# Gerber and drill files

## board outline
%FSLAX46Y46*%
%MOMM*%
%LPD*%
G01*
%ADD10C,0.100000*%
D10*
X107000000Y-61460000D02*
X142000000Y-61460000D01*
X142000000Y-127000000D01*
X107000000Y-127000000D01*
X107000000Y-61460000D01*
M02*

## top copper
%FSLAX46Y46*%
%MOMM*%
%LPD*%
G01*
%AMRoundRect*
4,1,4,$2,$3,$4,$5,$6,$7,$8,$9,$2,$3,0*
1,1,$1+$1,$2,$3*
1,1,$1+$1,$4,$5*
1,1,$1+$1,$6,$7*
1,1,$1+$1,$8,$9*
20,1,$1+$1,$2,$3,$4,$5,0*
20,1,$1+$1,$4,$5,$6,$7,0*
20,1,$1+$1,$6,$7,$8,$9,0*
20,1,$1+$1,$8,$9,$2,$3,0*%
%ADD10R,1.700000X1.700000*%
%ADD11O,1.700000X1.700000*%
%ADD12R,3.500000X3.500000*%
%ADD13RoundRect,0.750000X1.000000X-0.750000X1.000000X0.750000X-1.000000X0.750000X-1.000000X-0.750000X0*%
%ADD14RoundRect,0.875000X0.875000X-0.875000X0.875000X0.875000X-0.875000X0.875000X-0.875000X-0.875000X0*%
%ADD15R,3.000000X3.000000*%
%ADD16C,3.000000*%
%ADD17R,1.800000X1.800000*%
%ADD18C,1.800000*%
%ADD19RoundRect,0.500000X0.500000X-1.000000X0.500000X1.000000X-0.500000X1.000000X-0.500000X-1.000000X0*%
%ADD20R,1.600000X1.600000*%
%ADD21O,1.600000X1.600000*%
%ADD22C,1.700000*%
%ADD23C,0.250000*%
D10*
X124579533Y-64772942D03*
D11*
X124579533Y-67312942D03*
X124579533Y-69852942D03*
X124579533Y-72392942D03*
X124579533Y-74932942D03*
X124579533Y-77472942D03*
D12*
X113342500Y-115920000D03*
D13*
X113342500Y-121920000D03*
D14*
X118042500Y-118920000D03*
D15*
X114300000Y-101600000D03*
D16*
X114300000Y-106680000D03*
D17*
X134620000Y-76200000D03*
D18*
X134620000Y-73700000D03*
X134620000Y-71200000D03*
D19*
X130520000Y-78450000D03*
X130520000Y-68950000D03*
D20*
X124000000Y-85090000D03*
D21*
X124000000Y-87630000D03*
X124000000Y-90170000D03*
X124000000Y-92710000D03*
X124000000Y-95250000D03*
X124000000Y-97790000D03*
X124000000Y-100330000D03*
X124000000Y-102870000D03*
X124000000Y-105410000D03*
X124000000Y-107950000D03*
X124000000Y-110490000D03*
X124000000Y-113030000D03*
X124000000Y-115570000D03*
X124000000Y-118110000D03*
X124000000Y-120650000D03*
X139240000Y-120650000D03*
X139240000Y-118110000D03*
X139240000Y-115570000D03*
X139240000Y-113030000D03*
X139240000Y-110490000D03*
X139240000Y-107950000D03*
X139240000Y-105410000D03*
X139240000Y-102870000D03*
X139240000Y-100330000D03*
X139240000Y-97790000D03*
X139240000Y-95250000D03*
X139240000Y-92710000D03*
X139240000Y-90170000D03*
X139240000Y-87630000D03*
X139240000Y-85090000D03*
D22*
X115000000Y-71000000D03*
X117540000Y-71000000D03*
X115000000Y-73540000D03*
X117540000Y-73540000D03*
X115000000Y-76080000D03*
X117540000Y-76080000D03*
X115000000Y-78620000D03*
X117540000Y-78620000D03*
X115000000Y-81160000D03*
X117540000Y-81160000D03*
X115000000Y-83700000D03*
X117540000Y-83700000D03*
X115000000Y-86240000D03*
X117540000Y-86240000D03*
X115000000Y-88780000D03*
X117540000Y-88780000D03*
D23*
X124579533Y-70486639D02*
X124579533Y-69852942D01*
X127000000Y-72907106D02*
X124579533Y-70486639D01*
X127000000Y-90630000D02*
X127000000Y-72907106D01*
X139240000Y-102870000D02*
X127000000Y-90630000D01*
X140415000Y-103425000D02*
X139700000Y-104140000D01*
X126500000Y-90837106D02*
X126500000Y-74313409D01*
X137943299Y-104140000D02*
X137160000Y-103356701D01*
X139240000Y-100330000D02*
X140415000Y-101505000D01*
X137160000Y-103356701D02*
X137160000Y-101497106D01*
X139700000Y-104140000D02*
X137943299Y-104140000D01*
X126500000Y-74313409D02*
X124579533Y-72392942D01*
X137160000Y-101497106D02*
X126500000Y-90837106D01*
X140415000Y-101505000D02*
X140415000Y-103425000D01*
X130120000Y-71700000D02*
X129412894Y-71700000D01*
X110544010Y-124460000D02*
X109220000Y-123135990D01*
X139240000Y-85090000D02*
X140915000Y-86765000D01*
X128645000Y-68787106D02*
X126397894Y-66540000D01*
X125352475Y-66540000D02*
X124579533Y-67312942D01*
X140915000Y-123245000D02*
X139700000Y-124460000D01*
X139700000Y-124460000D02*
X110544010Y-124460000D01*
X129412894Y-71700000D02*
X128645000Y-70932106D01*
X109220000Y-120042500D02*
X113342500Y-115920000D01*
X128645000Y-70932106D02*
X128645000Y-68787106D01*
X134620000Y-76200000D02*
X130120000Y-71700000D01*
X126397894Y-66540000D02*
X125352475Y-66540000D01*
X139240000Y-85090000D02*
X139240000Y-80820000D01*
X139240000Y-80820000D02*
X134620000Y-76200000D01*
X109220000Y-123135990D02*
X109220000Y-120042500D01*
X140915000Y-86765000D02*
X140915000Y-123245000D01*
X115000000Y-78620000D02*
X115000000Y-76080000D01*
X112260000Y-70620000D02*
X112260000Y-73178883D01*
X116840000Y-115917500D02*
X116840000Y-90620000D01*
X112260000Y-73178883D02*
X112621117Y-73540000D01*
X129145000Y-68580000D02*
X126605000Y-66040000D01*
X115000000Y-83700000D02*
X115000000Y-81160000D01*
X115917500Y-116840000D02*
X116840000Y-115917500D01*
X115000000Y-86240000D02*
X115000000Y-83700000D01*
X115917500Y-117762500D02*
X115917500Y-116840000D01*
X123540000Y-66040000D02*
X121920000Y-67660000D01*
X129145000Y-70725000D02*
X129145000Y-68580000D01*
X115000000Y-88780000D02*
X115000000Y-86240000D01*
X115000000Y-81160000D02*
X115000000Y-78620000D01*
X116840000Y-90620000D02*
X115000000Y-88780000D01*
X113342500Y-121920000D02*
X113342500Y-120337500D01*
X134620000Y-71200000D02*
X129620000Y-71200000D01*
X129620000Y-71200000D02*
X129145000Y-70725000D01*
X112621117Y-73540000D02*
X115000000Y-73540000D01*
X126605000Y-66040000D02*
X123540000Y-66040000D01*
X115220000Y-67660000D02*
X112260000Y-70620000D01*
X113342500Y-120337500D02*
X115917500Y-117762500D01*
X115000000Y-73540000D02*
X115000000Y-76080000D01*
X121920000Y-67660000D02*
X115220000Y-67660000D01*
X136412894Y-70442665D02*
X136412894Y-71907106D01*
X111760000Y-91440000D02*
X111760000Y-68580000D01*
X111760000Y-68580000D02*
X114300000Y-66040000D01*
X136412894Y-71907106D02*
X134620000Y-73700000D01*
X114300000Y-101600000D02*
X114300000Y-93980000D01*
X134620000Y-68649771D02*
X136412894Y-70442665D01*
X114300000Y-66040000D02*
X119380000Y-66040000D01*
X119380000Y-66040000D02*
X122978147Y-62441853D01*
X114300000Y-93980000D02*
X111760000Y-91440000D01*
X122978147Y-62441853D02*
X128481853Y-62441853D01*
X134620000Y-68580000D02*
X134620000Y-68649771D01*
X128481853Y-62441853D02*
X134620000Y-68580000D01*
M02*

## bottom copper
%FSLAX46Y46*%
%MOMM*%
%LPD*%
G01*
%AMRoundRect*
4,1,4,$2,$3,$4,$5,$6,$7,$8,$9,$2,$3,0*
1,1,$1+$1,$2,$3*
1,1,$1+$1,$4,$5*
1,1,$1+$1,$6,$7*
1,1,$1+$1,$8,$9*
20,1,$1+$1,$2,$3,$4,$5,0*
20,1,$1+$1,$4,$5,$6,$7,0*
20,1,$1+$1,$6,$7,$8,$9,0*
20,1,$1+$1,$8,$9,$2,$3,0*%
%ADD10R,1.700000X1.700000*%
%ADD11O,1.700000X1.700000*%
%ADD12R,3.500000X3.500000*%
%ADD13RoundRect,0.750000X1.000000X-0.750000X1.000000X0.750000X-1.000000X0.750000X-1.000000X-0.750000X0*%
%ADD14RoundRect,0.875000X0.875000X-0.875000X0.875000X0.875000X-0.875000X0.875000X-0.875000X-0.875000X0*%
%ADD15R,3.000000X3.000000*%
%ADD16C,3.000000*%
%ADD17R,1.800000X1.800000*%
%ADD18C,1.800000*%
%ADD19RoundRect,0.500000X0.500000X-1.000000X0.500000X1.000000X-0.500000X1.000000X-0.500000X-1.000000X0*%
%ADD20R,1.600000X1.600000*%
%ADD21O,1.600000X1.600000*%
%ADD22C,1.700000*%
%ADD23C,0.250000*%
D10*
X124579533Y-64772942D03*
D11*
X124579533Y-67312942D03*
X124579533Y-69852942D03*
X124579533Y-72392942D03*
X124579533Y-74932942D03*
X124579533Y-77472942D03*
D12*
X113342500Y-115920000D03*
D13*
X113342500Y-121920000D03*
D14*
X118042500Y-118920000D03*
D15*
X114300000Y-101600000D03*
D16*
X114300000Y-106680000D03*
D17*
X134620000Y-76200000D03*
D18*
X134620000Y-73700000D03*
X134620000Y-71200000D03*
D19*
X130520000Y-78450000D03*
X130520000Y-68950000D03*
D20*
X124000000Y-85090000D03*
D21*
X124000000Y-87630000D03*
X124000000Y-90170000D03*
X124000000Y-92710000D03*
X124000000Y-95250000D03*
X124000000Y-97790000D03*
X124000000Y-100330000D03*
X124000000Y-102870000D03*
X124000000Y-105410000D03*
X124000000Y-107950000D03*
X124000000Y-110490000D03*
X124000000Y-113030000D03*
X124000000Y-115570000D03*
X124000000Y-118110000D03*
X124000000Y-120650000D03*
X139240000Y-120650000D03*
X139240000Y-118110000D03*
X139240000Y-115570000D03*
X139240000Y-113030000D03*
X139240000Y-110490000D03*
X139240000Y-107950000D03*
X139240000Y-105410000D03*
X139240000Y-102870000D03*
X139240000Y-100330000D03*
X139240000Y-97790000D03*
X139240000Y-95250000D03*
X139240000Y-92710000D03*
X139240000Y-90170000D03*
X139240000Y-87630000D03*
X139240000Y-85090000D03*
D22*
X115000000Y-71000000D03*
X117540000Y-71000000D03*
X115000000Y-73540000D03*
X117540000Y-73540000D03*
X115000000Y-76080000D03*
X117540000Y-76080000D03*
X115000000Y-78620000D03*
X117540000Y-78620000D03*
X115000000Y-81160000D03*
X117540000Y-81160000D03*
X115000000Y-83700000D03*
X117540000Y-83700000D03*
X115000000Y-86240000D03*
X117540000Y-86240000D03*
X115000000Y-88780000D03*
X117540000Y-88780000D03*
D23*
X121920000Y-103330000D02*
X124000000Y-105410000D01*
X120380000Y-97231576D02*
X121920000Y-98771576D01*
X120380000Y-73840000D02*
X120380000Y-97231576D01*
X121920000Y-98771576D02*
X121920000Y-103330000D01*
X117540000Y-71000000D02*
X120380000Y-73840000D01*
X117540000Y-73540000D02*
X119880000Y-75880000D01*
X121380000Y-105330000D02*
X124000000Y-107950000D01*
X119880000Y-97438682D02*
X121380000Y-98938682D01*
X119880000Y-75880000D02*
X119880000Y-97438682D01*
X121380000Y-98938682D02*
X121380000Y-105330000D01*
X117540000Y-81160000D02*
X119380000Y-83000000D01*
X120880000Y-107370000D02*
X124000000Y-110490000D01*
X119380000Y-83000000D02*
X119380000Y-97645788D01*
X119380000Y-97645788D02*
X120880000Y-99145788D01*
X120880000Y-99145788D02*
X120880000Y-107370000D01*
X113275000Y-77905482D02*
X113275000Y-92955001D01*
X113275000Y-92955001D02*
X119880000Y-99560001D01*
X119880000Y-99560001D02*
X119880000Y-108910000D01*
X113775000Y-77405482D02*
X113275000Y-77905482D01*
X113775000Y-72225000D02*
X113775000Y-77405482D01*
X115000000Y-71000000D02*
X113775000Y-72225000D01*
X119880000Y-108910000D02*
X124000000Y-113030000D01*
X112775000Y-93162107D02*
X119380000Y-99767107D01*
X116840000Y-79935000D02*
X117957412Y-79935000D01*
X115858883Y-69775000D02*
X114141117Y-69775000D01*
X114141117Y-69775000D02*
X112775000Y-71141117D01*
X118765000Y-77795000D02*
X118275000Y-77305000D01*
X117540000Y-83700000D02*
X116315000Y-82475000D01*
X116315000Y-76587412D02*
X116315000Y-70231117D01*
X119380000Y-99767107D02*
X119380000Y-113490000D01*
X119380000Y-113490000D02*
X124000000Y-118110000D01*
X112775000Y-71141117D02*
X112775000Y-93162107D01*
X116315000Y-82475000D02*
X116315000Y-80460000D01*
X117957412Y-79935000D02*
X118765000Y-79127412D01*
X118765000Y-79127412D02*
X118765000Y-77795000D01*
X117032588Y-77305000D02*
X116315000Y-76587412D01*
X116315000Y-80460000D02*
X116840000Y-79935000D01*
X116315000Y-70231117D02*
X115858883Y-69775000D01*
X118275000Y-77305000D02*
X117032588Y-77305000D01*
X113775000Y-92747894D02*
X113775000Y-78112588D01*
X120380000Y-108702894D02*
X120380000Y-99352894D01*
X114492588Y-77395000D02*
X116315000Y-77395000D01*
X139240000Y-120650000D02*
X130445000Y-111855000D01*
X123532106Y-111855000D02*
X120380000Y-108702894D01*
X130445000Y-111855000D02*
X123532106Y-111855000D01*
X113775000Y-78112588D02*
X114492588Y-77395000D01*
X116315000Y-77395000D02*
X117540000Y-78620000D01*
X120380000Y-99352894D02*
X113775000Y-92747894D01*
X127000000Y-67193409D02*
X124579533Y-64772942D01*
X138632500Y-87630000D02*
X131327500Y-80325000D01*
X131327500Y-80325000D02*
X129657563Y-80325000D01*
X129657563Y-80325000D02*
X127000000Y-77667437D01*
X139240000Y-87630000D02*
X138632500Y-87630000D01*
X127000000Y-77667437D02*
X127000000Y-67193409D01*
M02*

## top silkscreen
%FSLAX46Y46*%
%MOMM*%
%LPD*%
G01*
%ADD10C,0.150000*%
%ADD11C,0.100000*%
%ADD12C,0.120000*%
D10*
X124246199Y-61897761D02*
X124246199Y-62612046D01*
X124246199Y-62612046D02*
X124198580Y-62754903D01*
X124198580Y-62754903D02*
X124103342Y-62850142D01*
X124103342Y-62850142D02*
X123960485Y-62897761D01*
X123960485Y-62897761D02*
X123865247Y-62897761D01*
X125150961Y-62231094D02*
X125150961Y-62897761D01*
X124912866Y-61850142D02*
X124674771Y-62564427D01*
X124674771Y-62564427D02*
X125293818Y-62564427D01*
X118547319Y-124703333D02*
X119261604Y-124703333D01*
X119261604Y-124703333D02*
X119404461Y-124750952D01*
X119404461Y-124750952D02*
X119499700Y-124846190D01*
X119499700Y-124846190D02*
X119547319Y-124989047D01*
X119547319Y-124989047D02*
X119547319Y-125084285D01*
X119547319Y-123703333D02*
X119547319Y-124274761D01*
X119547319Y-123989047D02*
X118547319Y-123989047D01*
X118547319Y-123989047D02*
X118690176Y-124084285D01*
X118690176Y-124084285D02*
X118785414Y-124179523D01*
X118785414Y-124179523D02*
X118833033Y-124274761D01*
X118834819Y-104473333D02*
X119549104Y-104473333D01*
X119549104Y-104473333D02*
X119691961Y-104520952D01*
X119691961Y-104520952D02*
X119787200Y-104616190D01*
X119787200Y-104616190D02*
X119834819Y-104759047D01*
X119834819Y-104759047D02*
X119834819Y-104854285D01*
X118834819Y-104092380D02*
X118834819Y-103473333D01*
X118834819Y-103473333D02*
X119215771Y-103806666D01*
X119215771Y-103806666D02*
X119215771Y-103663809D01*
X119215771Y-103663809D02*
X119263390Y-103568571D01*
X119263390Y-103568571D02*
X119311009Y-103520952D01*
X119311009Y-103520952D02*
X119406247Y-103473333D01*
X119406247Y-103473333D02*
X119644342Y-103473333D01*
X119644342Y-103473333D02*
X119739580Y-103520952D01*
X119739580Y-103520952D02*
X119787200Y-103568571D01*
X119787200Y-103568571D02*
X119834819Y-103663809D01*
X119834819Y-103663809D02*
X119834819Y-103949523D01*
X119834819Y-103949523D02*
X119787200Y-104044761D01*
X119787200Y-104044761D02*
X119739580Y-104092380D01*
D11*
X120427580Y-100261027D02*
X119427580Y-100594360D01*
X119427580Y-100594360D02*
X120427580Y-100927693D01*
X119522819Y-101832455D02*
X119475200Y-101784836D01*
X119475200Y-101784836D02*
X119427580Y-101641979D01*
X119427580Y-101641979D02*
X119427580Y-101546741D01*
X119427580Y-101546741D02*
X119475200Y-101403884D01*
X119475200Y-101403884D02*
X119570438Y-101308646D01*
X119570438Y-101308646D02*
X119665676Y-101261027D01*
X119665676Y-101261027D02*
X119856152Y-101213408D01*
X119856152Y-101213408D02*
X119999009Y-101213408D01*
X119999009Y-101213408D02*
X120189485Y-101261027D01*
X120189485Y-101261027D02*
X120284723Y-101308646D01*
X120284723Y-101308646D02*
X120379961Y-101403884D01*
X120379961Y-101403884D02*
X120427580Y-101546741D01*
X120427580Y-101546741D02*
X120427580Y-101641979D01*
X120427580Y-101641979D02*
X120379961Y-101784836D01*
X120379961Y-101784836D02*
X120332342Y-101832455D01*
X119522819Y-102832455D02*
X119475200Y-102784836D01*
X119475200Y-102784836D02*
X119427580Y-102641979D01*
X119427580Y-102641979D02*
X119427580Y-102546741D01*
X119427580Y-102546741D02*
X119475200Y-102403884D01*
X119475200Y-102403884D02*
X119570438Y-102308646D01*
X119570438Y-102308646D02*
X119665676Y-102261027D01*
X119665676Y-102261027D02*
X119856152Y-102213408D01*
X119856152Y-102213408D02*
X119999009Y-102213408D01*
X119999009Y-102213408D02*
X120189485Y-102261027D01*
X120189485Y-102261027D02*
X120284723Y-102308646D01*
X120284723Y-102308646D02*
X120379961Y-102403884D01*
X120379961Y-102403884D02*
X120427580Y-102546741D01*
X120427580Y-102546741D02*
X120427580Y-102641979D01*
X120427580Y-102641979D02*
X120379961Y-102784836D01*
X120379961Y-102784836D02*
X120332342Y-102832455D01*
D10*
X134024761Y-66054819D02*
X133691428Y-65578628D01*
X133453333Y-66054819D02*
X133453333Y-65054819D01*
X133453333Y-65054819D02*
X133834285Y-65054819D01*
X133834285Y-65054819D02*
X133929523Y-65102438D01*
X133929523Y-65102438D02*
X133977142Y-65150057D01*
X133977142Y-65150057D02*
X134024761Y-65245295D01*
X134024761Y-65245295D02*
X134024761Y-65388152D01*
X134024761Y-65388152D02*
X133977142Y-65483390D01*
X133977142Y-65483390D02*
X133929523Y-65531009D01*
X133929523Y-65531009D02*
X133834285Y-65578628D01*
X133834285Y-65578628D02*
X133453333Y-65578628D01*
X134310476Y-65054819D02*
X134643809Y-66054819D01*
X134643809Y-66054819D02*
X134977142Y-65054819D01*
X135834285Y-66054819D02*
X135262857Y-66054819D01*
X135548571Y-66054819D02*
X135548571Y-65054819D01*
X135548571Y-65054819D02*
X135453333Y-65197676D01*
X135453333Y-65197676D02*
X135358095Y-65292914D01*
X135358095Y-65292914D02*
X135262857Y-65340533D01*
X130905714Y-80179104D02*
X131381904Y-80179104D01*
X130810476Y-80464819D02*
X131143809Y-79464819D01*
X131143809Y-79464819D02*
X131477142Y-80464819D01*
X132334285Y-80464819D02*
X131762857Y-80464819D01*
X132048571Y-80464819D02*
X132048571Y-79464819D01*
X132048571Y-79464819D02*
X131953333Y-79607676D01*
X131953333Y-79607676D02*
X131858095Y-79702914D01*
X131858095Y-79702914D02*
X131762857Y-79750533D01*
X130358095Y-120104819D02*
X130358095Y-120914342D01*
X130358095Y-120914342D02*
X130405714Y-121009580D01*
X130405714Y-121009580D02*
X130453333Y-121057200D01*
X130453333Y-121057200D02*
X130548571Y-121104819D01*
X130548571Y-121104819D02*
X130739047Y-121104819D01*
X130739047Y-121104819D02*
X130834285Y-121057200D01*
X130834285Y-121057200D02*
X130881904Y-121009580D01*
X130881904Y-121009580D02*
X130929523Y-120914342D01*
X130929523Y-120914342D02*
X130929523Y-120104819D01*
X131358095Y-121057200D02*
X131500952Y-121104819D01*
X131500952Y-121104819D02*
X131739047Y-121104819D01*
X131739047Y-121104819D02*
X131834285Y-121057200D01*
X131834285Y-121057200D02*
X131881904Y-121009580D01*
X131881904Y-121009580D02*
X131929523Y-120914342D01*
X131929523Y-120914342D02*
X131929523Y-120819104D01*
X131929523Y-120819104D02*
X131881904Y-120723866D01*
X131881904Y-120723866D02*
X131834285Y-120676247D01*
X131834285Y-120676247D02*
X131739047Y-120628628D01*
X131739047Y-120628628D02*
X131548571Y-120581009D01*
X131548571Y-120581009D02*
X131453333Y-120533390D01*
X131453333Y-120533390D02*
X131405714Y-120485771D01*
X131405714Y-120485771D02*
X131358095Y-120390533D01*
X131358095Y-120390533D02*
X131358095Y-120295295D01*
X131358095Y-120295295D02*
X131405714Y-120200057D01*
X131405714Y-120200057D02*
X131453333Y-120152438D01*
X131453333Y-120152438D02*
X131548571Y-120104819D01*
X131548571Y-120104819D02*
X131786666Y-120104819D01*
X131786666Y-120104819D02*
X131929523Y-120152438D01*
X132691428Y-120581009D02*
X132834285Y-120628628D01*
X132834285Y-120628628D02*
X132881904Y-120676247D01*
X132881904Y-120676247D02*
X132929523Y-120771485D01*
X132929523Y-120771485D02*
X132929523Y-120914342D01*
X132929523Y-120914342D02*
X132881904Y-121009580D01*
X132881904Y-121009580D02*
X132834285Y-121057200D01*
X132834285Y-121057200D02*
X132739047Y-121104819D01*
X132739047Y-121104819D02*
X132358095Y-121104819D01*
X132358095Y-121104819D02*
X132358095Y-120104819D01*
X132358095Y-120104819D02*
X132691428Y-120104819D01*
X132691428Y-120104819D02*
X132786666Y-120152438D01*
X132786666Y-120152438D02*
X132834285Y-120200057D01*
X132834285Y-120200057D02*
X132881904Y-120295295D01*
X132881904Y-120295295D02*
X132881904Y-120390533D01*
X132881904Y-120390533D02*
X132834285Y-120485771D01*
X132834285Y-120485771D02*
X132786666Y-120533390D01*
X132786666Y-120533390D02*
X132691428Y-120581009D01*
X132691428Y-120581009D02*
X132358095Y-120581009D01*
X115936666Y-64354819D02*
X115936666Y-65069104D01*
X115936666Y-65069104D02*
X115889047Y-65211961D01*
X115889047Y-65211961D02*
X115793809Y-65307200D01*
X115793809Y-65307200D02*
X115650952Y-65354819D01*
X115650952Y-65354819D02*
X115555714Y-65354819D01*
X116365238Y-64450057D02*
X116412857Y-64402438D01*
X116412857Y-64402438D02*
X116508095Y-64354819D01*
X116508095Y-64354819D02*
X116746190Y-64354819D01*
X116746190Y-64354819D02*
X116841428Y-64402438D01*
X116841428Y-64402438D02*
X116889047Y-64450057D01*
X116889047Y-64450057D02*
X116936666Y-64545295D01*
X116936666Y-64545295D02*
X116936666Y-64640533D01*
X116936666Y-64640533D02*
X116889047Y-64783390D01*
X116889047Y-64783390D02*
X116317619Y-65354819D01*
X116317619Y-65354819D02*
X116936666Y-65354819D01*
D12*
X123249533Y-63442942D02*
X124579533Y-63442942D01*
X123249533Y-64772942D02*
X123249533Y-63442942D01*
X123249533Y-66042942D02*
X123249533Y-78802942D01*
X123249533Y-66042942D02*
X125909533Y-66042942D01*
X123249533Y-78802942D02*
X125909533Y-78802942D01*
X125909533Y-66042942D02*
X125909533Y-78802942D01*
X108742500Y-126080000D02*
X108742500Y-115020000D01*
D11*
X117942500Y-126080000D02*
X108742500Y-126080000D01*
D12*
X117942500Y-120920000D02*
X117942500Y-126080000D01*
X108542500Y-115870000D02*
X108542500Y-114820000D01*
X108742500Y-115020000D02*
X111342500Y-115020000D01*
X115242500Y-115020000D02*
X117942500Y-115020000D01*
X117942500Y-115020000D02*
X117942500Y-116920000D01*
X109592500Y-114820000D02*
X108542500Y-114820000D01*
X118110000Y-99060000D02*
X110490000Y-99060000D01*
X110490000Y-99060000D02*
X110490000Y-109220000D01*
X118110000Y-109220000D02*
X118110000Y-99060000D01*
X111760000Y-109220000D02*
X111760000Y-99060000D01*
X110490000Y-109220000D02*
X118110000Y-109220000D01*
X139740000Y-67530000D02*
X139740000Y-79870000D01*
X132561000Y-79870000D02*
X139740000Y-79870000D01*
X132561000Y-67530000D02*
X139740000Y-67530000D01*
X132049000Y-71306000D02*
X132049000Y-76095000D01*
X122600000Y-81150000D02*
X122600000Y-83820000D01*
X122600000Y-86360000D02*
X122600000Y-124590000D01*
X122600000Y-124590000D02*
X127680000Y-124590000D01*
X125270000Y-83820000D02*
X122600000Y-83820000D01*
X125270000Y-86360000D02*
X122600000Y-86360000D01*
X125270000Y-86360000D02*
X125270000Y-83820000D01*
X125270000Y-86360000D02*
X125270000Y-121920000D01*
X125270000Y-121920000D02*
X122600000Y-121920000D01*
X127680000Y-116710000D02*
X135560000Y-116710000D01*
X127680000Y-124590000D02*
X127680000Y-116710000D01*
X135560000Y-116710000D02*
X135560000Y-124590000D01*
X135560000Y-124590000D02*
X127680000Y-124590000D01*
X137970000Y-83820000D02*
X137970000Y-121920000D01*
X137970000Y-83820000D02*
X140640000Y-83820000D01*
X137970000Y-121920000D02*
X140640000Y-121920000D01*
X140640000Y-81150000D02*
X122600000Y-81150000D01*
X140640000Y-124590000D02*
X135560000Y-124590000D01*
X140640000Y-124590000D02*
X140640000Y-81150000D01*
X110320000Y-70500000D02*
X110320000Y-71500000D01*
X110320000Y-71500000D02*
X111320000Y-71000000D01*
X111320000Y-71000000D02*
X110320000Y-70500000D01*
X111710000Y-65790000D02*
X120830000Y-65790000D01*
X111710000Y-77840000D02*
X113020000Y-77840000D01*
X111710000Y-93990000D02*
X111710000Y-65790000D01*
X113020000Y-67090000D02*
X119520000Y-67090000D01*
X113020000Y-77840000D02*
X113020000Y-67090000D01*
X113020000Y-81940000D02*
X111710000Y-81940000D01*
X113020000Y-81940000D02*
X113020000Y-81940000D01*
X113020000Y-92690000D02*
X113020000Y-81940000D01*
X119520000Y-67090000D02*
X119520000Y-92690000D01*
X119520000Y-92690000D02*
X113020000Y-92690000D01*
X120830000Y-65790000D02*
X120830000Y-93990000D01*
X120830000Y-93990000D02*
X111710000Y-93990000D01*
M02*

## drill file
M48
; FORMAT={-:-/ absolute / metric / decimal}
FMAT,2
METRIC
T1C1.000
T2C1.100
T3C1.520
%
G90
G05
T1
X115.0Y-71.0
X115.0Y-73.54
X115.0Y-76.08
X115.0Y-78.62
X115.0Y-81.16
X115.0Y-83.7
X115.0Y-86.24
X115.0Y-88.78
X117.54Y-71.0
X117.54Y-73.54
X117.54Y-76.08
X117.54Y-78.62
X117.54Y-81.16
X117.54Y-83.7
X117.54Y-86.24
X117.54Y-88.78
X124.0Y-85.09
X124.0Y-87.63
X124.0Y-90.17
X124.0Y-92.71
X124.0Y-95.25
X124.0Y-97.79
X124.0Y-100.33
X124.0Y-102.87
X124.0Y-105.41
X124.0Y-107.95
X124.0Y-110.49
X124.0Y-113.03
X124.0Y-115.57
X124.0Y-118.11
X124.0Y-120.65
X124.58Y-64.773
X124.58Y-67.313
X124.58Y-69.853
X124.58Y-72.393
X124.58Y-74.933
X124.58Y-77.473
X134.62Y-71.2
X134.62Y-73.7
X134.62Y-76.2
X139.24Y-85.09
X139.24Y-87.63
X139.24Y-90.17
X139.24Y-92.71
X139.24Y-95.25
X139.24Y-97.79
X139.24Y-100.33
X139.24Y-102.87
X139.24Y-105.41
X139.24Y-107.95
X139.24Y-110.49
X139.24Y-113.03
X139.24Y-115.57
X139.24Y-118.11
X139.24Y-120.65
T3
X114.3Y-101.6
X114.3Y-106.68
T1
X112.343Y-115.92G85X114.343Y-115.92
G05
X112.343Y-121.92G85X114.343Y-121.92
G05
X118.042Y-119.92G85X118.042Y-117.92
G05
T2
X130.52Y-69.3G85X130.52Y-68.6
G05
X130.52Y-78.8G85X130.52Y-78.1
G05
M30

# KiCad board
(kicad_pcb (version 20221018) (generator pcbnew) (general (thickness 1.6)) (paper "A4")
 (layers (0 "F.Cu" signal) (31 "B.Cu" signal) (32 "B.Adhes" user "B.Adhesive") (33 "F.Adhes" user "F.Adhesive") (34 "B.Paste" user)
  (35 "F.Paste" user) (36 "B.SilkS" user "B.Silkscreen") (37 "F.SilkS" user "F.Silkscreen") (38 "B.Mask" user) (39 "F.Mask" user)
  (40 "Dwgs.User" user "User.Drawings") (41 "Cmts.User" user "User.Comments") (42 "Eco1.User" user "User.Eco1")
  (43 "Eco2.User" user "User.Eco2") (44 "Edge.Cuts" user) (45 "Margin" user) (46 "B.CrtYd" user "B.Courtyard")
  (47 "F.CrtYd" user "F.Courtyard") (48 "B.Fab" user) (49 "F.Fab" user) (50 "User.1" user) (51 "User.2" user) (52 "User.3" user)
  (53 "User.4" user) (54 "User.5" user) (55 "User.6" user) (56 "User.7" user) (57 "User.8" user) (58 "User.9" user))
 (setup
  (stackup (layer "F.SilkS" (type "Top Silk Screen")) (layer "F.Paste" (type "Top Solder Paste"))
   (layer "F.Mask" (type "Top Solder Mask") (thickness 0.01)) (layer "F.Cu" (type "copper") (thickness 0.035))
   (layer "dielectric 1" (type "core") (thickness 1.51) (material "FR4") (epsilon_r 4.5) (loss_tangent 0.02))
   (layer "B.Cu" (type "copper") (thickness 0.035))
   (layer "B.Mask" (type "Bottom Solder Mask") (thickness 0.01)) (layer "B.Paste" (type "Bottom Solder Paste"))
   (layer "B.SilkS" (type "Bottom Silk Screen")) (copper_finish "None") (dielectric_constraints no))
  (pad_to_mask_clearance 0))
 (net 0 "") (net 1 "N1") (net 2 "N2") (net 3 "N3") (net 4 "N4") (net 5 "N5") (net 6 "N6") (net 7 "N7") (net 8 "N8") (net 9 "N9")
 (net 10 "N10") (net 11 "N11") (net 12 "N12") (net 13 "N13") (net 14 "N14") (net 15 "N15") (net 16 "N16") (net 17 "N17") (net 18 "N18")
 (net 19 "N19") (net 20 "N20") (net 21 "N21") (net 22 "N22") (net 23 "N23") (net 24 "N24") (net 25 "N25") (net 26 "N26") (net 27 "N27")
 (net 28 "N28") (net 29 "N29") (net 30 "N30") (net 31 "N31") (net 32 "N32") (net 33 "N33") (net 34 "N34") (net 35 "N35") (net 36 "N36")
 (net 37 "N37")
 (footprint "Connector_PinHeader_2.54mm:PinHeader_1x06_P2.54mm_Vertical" (layer "F.Cu") (at 124.579533 64.772942)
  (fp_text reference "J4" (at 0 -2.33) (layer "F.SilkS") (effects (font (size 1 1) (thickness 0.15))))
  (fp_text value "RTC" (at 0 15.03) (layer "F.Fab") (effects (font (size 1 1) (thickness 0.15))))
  (fp_line (start -1.33 -1.33) (end 0 -1.33) (stroke (width 0.12) (type solid)) (layer "F.SilkS"))
  (fp_line (start -1.33 0) (end -1.33 -1.33) (stroke (width 0.12) (type solid)) (layer "F.SilkS"))
  (fp_line (start -1.33 1.27) (end -1.33 14.03) (stroke (width 0.12) (type solid)) (layer "F.SilkS"))
  (fp_line (start -1.33 1.27) (end 1.33 1.27) (stroke (width 0.12) (type solid)) (layer "F.SilkS"))
  (fp_line (start -1.33 14.03) (end 1.33 14.03) (stroke (width 0.12) (type solid)) (layer "F.SilkS"))
  (fp_line (start 1.33 1.27) (end 1.33 14.03) (stroke (width 0.12) (type solid)) (layer "F.SilkS"))
  (pad "1" thru_hole rect (at 0 0) (size 1.7 1.7) (drill 1) (layers "*.Cu" "*.Mask") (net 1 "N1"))
  (pad "2" thru_hole oval (at 0 2.54) (size 1.7 1.7) (drill 1) (layers "*.Cu" "*.Mask") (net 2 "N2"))
  (pad "3" thru_hole oval (at 0 5.08) (size 1.7 1.7) (drill 1) (layers "*.Cu" "*.Mask") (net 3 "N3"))
  (pad "4" thru_hole oval (at 0 7.62) (size 1.7 1.7) (drill 1) (layers "*.Cu" "*.Mask") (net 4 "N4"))
  (pad "5" thru_hole oval (at 0 10.16) (size 1.7 1.7) (drill 1) (layers "*.Cu" "*.Mask") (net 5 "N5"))
  (pad "6" thru_hole oval (at 0 12.7) (size 1.7 1.7) (drill 1) (layers "*.Cu" "*.Mask") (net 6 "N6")))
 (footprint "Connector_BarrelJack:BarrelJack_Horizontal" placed (layer "F.Cu") (at 113.3425 115.92 90)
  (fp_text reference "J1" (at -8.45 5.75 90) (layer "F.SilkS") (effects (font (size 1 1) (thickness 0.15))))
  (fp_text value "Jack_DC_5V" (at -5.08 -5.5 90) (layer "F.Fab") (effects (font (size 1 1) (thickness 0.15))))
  (fp_line (start -10.16 -4.6) (end 0.9 -4.6) (stroke (width 0.12) (type solid)) (layer "F.SilkS"))
  (fp_line (start -10.16 4.6) (end -10.16 -4.6) (stroke (width 0.1) (type default)) (layer "F.SilkS"))
  (fp_line (start -5 4.6) (end -10.16 4.6) (stroke (width 0.12) (type solid)) (layer "F.SilkS"))
  (fp_line (start 0.05 -4.8) (end 1.1 -4.8) (stroke (width 0.12) (type solid)) (layer "F.SilkS"))
  (fp_line (start 0.9 -4.6) (end 0.9 -2) (stroke (width 0.12) (type solid)) (layer "F.SilkS"))
  (fp_line (start 0.9 1.9) (end 0.9 4.6) (stroke (width 0.12) (type solid)) (layer "F.SilkS"))
  (fp_line (start 0.9 4.6) (end -1 4.6) (stroke (width 0.12) (type solid)) (layer "F.SilkS"))
  (fp_line (start 1.1 -3.75) (end 1.1 -4.8) (stroke (width 0.12) (type solid)) (layer "F.SilkS"))
  (pad "1" thru_hole rect (at 0 0 90) (size 3.5 3.5) (drill oval 1 3) (layers "*.Cu" "*.Mask") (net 2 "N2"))
  (pad "2" thru_hole roundrect (at -6 0 90) (size 3 3.5) (drill oval 1 3) (layers "*.Cu" "*.Mask") (roundrect_rratio 0.25) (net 1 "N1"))
  (pad "3" thru_hole roundrect (at -3 4.7 90) (size 3.5 3.5) (drill oval 3 1) (layers "*.Cu" "*.Mask") (roundrect_rratio 0.25)))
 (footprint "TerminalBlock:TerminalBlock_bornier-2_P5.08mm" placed (layer "F.Cu") (at 114.3 101.6 -90)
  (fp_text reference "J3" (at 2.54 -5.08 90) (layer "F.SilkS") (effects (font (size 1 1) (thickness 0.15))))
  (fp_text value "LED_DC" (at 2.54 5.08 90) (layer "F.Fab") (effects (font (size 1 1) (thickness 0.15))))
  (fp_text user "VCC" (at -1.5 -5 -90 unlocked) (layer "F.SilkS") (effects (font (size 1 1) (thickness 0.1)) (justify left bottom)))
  (fp_line (start -2.54 -3.81) (end -2.54 3.81) (stroke (width 0.12) (type solid)) (layer "F.SilkS"))
  (fp_line (start -2.54 3.81) (end 7.62 3.81) (stroke (width 0.12) (type solid)) (layer "F.SilkS"))
  (fp_line (start 7.62 -3.81) (end -2.54 -3.81) (stroke (width 0.12) (type solid)) (layer "F.SilkS"))
  (fp_line (start 7.62 2.54) (end -2.54 2.54) (stroke (width 0.12) (type solid)) (layer "F.SilkS"))
  (fp_line (start 7.62 3.81) (end 7.62 -3.81) (stroke (width 0.12) (type solid)) (layer "F.SilkS"))
  (pad "1" thru_hole rect (at 0 0 270) (size 3 3) (drill 1.52) (layers "*.Cu" "*.Mask") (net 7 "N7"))
  (pad "2" thru_hole circle (at 5.08 0 270) (size 3 3) (drill 1.52) (layers "*.Cu" "*.Mask") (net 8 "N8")))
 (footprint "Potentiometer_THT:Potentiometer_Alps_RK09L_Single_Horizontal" (layer "F.Cu") (at 134.62 76.2 180)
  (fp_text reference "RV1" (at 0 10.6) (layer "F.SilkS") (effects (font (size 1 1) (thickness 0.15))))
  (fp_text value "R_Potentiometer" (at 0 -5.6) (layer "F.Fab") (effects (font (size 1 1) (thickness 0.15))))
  (fp_line (start -5.12 8.67) (end -5.12 -3.67) (stroke (width 0.12) (type solid)) (layer "F.SilkS"))
  (fp_line (start 2.059 -3.67) (end -5.12 -3.67) (stroke (width 0.12) (type solid)) (layer "F.SilkS"))
  (fp_line (start 2.059 8.67) (end -5.12 8.67) (stroke (width 0.12) (type solid)) (layer "F.SilkS"))
  (fp_line (start 2.571 4.894) (end 2.571 0.105) (stroke (width 0.12) (type solid)) (layer "F.SilkS"))
  (pad "1" thru_hole rect (at 0 0) (size 1.8 1.8) (drill 1) (layers "*.Cu" "*.Mask") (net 2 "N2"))
  (pad "2" thru_hole circle (at 0 2.5) (size 1.8 1.8) (drill 1) (layers "*.Cu" "*.Mask") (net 7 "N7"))
  (pad "3" thru_hole circle (at 0 5) (size 1.8 1.8) (drill 1) (layers "*.Cu" "*.Mask") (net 1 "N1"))
  (pad "MP" thru_hole roundrect (at 4.1 -2.25 90) (size 3 2) (drill oval 1.8 1.1) (layers "*.Cu" "*.Mask") (roundrect_rratio 0.25))
  (pad "MP" thru_hole roundrect (at 4.1 7.25 90) (size 3 2) (drill oval 1.8 1.1) (layers "*.Cu" "*.Mask") (roundrect_rratio 0.25)))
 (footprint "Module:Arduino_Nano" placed (layer "F.Cu") (at 124 85.09)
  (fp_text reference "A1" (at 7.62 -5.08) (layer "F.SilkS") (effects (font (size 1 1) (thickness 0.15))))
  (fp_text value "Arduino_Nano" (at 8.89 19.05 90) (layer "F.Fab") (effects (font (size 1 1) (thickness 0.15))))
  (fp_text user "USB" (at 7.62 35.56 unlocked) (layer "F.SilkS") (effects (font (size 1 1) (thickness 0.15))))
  (fp_line (start -1.4 -3.94) (end -1.4 -1.27) (stroke (width 0.12) (type solid)) (layer "F.SilkS"))
  (fp_line (start -1.4 1.27) (end -1.4 39.5) (stroke (width 0.12) (type solid)) (layer "F.SilkS"))
  (fp_line (start -1.4 39.5) (end 3.68 39.5) (stroke (width 0.12) (type solid)) (layer "F.SilkS"))
  (fp_line (start 1.27 -1.27) (end -1.4 -1.27) (stroke (width 0.12) (type solid)) (layer "F.SilkS"))
  (fp_line (start 1.27 1.27) (end -1.4 1.27) (stroke (width 0.12) (type solid)) (layer "F.SilkS"))
  (fp_line (start 1.27 1.27) (end 1.27 -1.27) (stroke (width 0.12) (type solid)) (layer "F.SilkS"))
  (fp_line (start 1.27 1.27) (end 1.27 36.83) (stroke (width 0.12) (type solid)) (layer "F.SilkS"))
  (fp_line (start 1.27 36.83) (end -1.4 36.83) (stroke (width 0.12) (type solid)) (layer "F.SilkS"))
  (fp_line (start 3.68 31.62) (end 11.56 31.62) (stroke (width 0.12) (type solid)) (layer "F.SilkS"))
  (fp_line (start 3.68 39.5) (end 3.68 31.62) (stroke (width 0.12) (type solid)) (layer "F.SilkS"))
  (fp_line (start 11.56 31.62) (end 11.56 39.5) (stroke (width 0.12) (type solid)) (layer "F.SilkS"))
  (fp_line (start 11.56 39.5) (end 3.68 39.5) (stroke (width 0.12) (type solid)) (layer "F.SilkS"))
  (fp_line (start 13.97 -1.27) (end 13.97 36.83) (stroke (width 0.12) (type solid)) (layer "F.SilkS"))
  (fp_line (start 13.97 -1.27) (end 16.64 -1.27) (stroke (width 0.12) (type solid)) (layer "F.SilkS"))
  (fp_line (start 13.97 36.83) (end 16.64 36.83) (stroke (width 0.12) (type solid)) (layer "F.SilkS"))
  (fp_line (start 16.64 -3.94) (end -1.4 -3.94) (stroke (width 0.12) (type solid)) (layer "F.SilkS"))
  (fp_line (start 16.64 39.5) (end 11.56 39.5) (stroke (width 0.12) (type solid)) (layer "F.SilkS"))
  (fp_line (start 16.64 39.5) (end 16.64 -3.94) (stroke (width 0.12) (type solid)) (layer "F.SilkS"))
  (pad "1" thru_hole rect (at 0 0) (size 1.6 1.6) (drill 1) (layers "*.Cu" "*.Mask") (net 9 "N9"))
  (pad "2" thru_hole oval (at 0 2.54) (size 1.6 1.6) (drill 1) (layers "*.Cu" "*.Mask") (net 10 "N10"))
  (pad "3" thru_hole oval (at 0 5.08) (size 1.6 1.6) (drill 1) (layers "*.Cu" "*.Mask") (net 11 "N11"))
  (pad "4" thru_hole oval (at 0 7.62) (size 1.6 1.6) (drill 1) (layers "*.Cu" "*.Mask") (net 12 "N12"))
  (pad "5" thru_hole oval (at 0 10.16) (size 1.6 1.6) (drill 1) (layers "*.Cu" "*.Mask") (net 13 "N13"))
  (pad "6" thru_hole oval (at 0 12.7) (size 1.6 1.6) (drill 1) (layers "*.Cu" "*.Mask") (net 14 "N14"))
  (pad "7" thru_hole oval (at 0 15.24) (size 1.6 1.6) (drill 1) (layers "*.Cu" "*.Mask") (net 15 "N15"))
  (pad "8" thru_hole oval (at 0 17.78) (size 1.6 1.6) (drill 1) (layers "*.Cu" "*.Mask") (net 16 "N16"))
  (pad "9" thru_hole oval (at 0 20.32) (size 1.6 1.6) (drill 1) (layers "*.Cu" "*.Mask") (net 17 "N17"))
  (pad "10" thru_hole oval (at 0 22.86) (size 1.6 1.6) (drill 1) (layers "*.Cu" "*.Mask") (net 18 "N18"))
  (pad "11" thru_hole oval (at 0 25.4) (size 1.6 1.6) (drill 1) (layers "*.Cu" "*.Mask") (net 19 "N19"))
  (pad "12" thru_hole oval (at 0 27.94) (size 1.6 1.6) (drill 1) (layers "*.Cu" "*.Mask") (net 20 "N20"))
  (pad "13" thru_hole oval (at 0 30.48) (size 1.6 1.6) (drill 1) (layers "*.Cu" "*.Mask") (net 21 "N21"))
  (pad "14" thru_hole oval (at 0 33.02) (size 1.6 1.6) (drill 1) (layers "*.Cu" "*.Mask") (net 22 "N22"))
  (pad "15" thru_hole oval (at 0 35.56) (size 1.6 1.6) (drill 1) (layers "*.Cu" "*.Mask") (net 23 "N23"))
  (pad "16" thru_hole oval (at 15.24 35.56) (size 1.6 1.6) (drill 1) (layers "*.Cu" "*.Mask") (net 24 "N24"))
  (pad "17" thru_hole oval (at 15.24 33.02) (size 1.6 1.6) (drill 1) (layers "*.Cu" "*.Mask") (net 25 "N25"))
  (pad "18" thru_hole oval (at 15.24 30.48) (size 1.6 1.6) (drill 1) (layers "*.Cu" "*.Mask") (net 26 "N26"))
  (pad "19" thru_hole oval (at 15.24 27.94) (size 1.6 1.6) (drill 1) (layers "*.Cu" "*.Mask") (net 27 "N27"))
  (pad "20" thru_hole oval (at 15.24 25.4) (size 1.6 1.6) (drill 1) (layers "*.Cu" "*.Mask") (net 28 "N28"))
  (pad "21" thru_hole oval (at 15.24 22.86) (size 1.6 1.6) (drill 1) (layers "*.Cu" "*.Mask") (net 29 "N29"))
  (pad "22" thru_hole oval (at 15.24 20.32) (size 1.6 1.6) (drill 1) (layers "*.Cu" "*.Mask") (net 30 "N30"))
  (pad "23" thru_hole oval (at 15.24 17.78) (size 1.6 1.6) (drill 1) (layers "*.Cu" "*.Mask") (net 3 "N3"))
  (pad "24" thru_hole oval (at 15.24 15.24) (size 1.6 1.6) (drill 1) (layers "*.Cu" "*.Mask") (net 4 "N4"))
  (pad "25" thru_hole oval (at 15.24 12.7) (size 1.6 1.6) (drill 1) (layers "*.Cu" "*.Mask") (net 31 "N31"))
  (pad "26" thru_hole oval (at 15.24 10.16) (size 1.6 1.6) (drill 1) (layers "*.Cu" "*.Mask") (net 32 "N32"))
  (pad "27" thru_hole oval (at 15.24 7.62) (size 1.6 1.6) (drill 1) (layers "*.Cu" "*.Mask") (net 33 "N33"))
  (pad "28" thru_hole oval (at 15.24 5.08) (size 1.6 1.6) (drill 1) (layers "*.Cu" "*.Mask") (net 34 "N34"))
  (pad "29" thru_hole oval (at 15.24 2.54) (size 1.6 1.6) (drill 1) (layers "*.Cu" "*.Mask") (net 1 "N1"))
  (pad "30" thru_hole oval (at 15.24 0) (size 1.6 1.6) (drill 1) (layers "*.Cu" "*.Mask") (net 2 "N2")))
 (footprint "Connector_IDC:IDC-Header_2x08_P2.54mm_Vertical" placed (layer "F.Cu") (at 115 71)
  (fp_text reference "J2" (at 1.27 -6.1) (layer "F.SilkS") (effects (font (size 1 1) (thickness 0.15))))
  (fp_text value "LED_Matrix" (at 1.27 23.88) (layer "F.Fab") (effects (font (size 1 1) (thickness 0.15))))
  (fp_line (start -4.68 -0.5) (end -4.68 0.5) (stroke (width 0.12) (type solid)) (layer "F.SilkS"))
  (fp_line (start -4.68 0.5) (end -3.68 0) (stroke (width 0.12) (type solid)) (layer "F.SilkS"))
  (fp_line (start -3.68 0) (end -4.68 -0.5) (stroke (width 0.12) (type solid)) (layer "F.SilkS"))
  (fp_line (start -3.29 -5.21) (end 5.83 -5.21) (stroke (width 0.12) (type solid)) (layer "F.SilkS"))
  (fp_line (start -3.29 6.84) (end -1.98 6.84) (stroke (width 0.12) (type solid)) (layer "F.SilkS"))
  (fp_line (start -3.29 22.99) (end -3.29 -5.21) (stroke (width 0.12) (type solid)) (layer "F.SilkS"))
  (fp_line (start -1.98 -3.91) (end 4.52 -3.91) (stroke (width 0.12) (type solid)) (layer "F.SilkS"))
  (fp_line (start -1.98 6.84) (end -1.98 -3.91) (stroke (width 0.12) (type solid)) (layer "F.SilkS"))
  (fp_line (start -1.98 10.94) (end -3.29 10.94) (stroke (width 0.12) (type solid)) (layer "F.SilkS"))
  (fp_line (start -1.98 10.94) (end -1.98 10.94) (stroke (width 0.12) (type solid)) (layer "F.SilkS"))
  (fp_line (start -1.98 21.69) (end -1.98 10.94) (stroke (width 0.12) (type solid)) (layer "F.SilkS"))
  (fp_line (start 4.52 -3.91) (end 4.52 21.69) (stroke (width 0.12) (type solid)) (layer "F.SilkS"))
  (fp_line (start 4.52 21.69) (end -1.98 21.69) (stroke (width 0.12) (type solid)) (layer "F.SilkS"))
  (fp_line (start 5.83 -5.21) (end 5.83 22.99) (stroke (width 0.12) (type solid)) (layer "F.SilkS"))
  (fp_line (start 5.83 22.99) (end -3.29 22.99) (stroke (width 0.12) (type solid)) (layer "F.SilkS"))
  (pad "1" thru_hole circle (at 0 0) (size 1.7 1.7) (drill 1) (layers "*.Cu" "*.Mask") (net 20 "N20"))
  (pad "2" thru_hole circle (at 2.54 0) (size 1.7 1.7) (drill 1) (layers "*.Cu" "*.Mask") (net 17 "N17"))
  (pad "3" thru_hole circle (at 0 2.54) (size 1.7 1.7) (drill 1) (layers "*.Cu" "*.Mask") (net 1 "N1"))
  (pad "4" thru_hole circle (at 2.54 2.54) (size 1.7 1.7) (drill 1) (layers "*.Cu" "*.Mask") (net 18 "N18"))
  (pad "5" thru_hole circle (at 0 5.08) (size 1.7 1.7) (drill 1) (layers "*.Cu" "*.Mask") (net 1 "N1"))
  (pad "6" thru_hole circle (at 2.54 5.08) (size 1.7 1.7) (drill 1) (layers "*.Cu" "*.Mask") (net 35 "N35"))
  (pad "7" thru_hole circle (at 0 7.62) (size 1.7 1.7) (drill 1) (layers "*.Cu" "*.Mask") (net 1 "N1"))
  (pad "8" thru_hole circle (at 2.54 7.62) (size 1.7 1.7) (drill 1) (layers "*.Cu" "*.Mask") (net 24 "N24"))
  (pad "9" thru_hole circle (at 0 10.16) (size 1.7 1.7) (drill 1) (layers "*.Cu" "*.Mask") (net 1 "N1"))
  (pad "10" thru_hole circle (at 2.54 10.16) (size 1.7 1.7) (drill 1) (layers "*.Cu" "*.Mask") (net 19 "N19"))
  (pad "11" thru_hole circle (at 0 12.7) (size 1.7 1.7) (drill 1) (layers "*.Cu" "*.Mask") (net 1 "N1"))
  (pad "12" thru_hole circle (at 2.54 12.7) (size 1.7 1.7) (drill 1) (layers "*.Cu" "*.Mask") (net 22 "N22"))
  (pad "13" thru_hole circle (at 0 15.24) (size 1.7 1.7) (drill 1) (layers "*.Cu" "*.Mask") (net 1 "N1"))
  (pad "14" thru_hole circle (at 2.54 15.24) (size 1.7 1.7) (drill 1) (layers "*.Cu" "*.Mask") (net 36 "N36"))
  (pad "15" thru_hole circle (at 0 17.78) (size 1.7 1.7) (drill 1) (layers "*.Cu" "*.Mask") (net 1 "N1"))
  (pad "16" thru_hole circle (at 2.54 17.78) (size 1.7 1.7) (drill 1) (layers "*.Cu" "*.Mask") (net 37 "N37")))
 (gr_rect (start 107 61.46) (end 142 127) (stroke (width 0.1) (type default)) (fill none) (layer "Edge.Cuts"))
 (segment (start 121.92 103.33) (end 124 105.41) (width 0.25) (layer "B.Cu") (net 17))
 (segment (start 120.38 97.231576) (end 121.92 98.771576) (width 0.25) (layer "B.Cu") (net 17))
 (segment (start 120.38 73.84) (end 120.38 97.231576) (width 0.25) (layer "B.Cu") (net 17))
 (segment (start 121.92 98.771576) (end 121.92 103.33) (width 0.25) (layer "B.Cu") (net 17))
 (segment (start 117.54 71) (end 120.38 73.84) (width 0.25) (layer "B.Cu") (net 17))
 (segment (start 117.54 73.54) (end 119.88 75.88) (width 0.25) (layer "B.Cu") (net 18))
 (segment (start 121.38 105.33) (end 124 107.95) (width 0.25) (layer "B.Cu") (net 18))
 (segment (start 119.88 97.438682) (end 121.38 98.938682) (width 0.25) (layer "B.Cu") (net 18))
 (segment (start 119.88 75.88) (end 119.88 97.438682) (width 0.25) (layer "B.Cu") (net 18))
 (segment (start 121.38 98.938682) (end 121.38 105.33) (width 0.25) (layer "B.Cu") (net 18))
 (segment (start 117.54 81.16) (end 119.38 83) (width 0.25) (layer "B.Cu") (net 19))
 (segment (start 120.88 107.37) (end 124 110.49) (width 0.25) (layer "B.Cu") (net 19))
 (segment (start 119.38 83) (end 119.38 97.645788) (width 0.25) (layer "B.Cu") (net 19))
 (segment (start 119.38 97.645788) (end 120.88 99.145788) (width 0.25) (layer "B.Cu") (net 19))
 (segment (start 120.88 99.145788) (end 120.88 107.37) (width 0.25) (layer "B.Cu") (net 19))
 (segment (start 113.275 77.905482) (end 113.275 92.955001) (width 0.25) (layer "B.Cu") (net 20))
 (segment (start 113.275 92.955001) (end 119.88 99.560001) (width 0.25) (layer "B.Cu") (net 20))
 (segment (start 119.88 99.560001) (end 119.88 108.91) (width 0.25) (layer "B.Cu") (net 20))
 (segment (start 113.775 77.405482) (end 113.275 77.905482) (width 0.25) (layer "B.Cu") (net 20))
 (segment (start 113.775 72.225) (end 113.775 77.405482) (width 0.25) (layer "B.Cu") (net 20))
 (segment (start 115 71) (end 113.775 72.225) (width 0.25) (layer "B.Cu") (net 20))
 (segment (start 119.88 108.91) (end 124 113.03) (width 0.25) (layer "B.Cu") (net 20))
 (segment (start 112.775 93.162107) (end 119.38 99.767107) (width 0.25) (layer "B.Cu") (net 22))
 (segment (start 116.84 79.935) (end 117.957412 79.935) (width 0.25) (layer "B.Cu") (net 22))
 (segment (start 115.858883 69.775) (end 114.141117 69.775) (width 0.25) (layer "B.Cu") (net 22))
 (segment (start 114.141117 69.775) (end 112.775 71.141117) (width 0.25) (layer "B.Cu") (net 22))
 (segment (start 118.765 77.795) (end 118.275 77.305) (width 0.25) (layer "B.Cu") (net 22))
 (segment (start 117.54 83.7) (end 116.315 82.475) (width 0.25) (layer "B.Cu") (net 22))
 (segment (start 116.315 76.587412) (end 116.315 70.231117) (width 0.25) (layer "B.Cu") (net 22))
 (segment (start 119.38 99.767107) (end 119.38 113.49) (width 0.25) (layer "B.Cu") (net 22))
 (segment (start 119.38 113.49) (end 124 118.11) (width 0.25) (layer "B.Cu") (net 22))
 (segment (start 112.775 71.141117) (end 112.775 93.162107) (width 0.25) (layer "B.Cu") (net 22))
 (segment (start 116.315 82.475) (end 116.315 80.46) (width 0.25) (layer "B.Cu") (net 22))
 (segment (start 117.957412 79.935) (end 118.765 79.127412) (width 0.25) (layer "B.Cu") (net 22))
 (segment (start 118.765 79.127412) (end 118.765 77.795) (width 0.25) (layer "B.Cu") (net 22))
 (segment (start 117.032588 77.305) (end 116.315 76.587412) (width 0.25) (layer "B.Cu") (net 22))
 (segment (start 116.315 80.46) (end 116.84 79.935) (width 0.25) (layer "B.Cu") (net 22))
 (segment (start 116.315 70.231117) (end 115.858883 69.775) (width 0.25) (layer "B.Cu") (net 22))
 (segment (start 118.275 77.305) (end 117.032588 77.305) (width 0.25) (layer "B.Cu") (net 22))
 (segment (start 113.775 92.747894) (end 113.775 78.112588) (width 0.25) (layer "B.Cu") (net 24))
 (segment (start 120.38 108.702894) (end 120.38 99.352894) (width 0.25) (layer "B.Cu") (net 24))
 (segment (start 114.492588 77.395) (end 116.315 77.395) (width 0.25) (layer "B.Cu") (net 24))
 (segment (start 139.24 120.65) (end 130.445 111.855) (width 0.25) (layer "B.Cu") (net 24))
 (segment (start 123.532106 111.855) (end 120.38 108.702894) (width 0.25) (layer "B.Cu") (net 24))
 (segment (start 130.445 111.855) (end 123.532106 111.855) (width 0.25) (layer "B.Cu") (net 24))
 (segment (start 113.775 78.112588) (end 114.492588 77.395) (width 0.25) (layer "B.Cu") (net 24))
 (segment (start 116.315 77.395) (end 117.54 78.62) (width 0.25) (layer "B.Cu") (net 24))
 (segment (start 120.38 99.352894) (end 113.775 92.747894) (width 0.25) (layer "B.Cu") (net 24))
 (segment (start 124.579533 70.486639) (end 124.579533 69.852942) (width 0.25) (layer "F.Cu") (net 3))
 (segment (start 127 72.907106) (end 124.579533 70.486639) (width 0.25) (layer "F.Cu") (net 3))
 (segment (start 127 90.63) (end 127 72.907106) (width 0.25) (layer "F.Cu") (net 3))
 (segment (start 139.24 102.87) (end 127 90.63) (width 0.25) (layer "F.Cu") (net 3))
 (segment (start 140.415 103.425) (end 139.7 104.14) (width 0.25) (layer "F.Cu") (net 4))
 (segment (start 126.5 90.837106) (end 126.5 74.313409) (width 0.25) (layer "F.Cu") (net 4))
 (segment (start 137.943299 104.14) (end 137.16 103.356701) (width 0.25) (layer "F.Cu") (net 4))
 (segment (start 139.24 100.33) (end 140.415 101.505) (width 0.25) (layer "F.Cu") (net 4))
 (segment (start 137.16 103.356701) (end 137.16 101.497106) (width 0.25) (layer "F.Cu") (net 4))
 (segment (start 139.7 104.14) (end 137.943299 104.14) (width 0.25) (layer "F.Cu") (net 4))
 (segment (start 126.5 74.313409) (end 124.579533 72.392942) (width 0.25) (layer "F.Cu") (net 4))
 (segment (start 137.16 101.497106) (end 126.5 90.837106) (width 0.25) (layer "F.Cu") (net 4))
 (segment (start 140.415 101.505) (end 140.415 103.425) (width 0.25) (layer "F.Cu") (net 4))
 (segment (start 130.12 71.7) (end 129.412894 71.7) (width 0.25) (layer "F.Cu") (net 2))
 (segment (start 110.54401 124.46) (end 109.22 123.13599) (width 0.25) (layer "F.Cu") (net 2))
 (segment (start 139.24 85.09) (end 140.915 86.765) (width 0.25) (layer "F.Cu") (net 2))
 (segment (start 128.645 68.787106) (end 126.397894 66.54) (width 0.25) (layer "F.Cu") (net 2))
 (segment (start 125.352475 66.54) (end 124.579533 67.312942) (width 0.25) (layer "F.Cu") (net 2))
 (segment (start 140.915 123.245) (end 139.7 124.46) (width 0.25) (layer "F.Cu") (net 2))
 (segment (start 139.7 124.46) (end 110.54401 124.46) (width 0.25) (layer "F.Cu") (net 2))
 (segment (start 129.412894 71.7) (end 128.645 70.932106) (width 0.25) (layer "F.Cu") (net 2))
 (segment (start 109.22 120.0425) (end 113.3425 115.92) (width 0.25) (layer "F.Cu") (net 2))
 (segment (start 128.645 70.932106) (end 128.645 68.787106) (width 0.25) (layer "F.Cu") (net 2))
 (segment (start 134.62 76.2) (end 130.12 71.7) (width 0.25) (layer "F.Cu") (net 2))
 (segment (start 126.397894 66.54) (end 125.352475 66.54) (width 0.25) (layer "F.Cu") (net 2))
 (segment (start 139.24 85.09) (end 139.24 80.82) (width 0.25) (layer "F.Cu") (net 2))
 (segment (start 139.24 80.82) (end 134.62 76.2) (width 0.25) (layer "F.Cu") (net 2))
 (segment (start 109.22 123.13599) (end 109.22 120.0425) (width 0.25) (layer "F.Cu") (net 2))
 (segment (start 140.915 86.765) (end 140.915 123.245) (width 0.25) (layer "F.Cu") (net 2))
 (segment (start 115 78.62) (end 115 76.08) (width 0.25) (layer "F.Cu") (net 1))
 (segment (start 112.26 70.62) (end 112.26 73.178883) (width 0.25) (layer "F.Cu") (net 1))
 (segment (start 116.84 115.9175) (end 116.84 90.62) (width 0.25) (layer "F.Cu") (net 1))
 (segment (start 112.26 73.178883) (end 112.621117 73.54) (width 0.25) (layer "F.Cu") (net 1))
 (segment (start 129.145 68.58) (end 126.605 66.04) (width 0.25) (layer "F.Cu") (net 1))
 (segment (start 115 83.7) (end 115 81.16) (width 0.25) (layer "F.Cu") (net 1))
 (segment (start 115.9175 116.84) (end 116.84 115.9175) (width 0.25) (layer "F.Cu") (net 1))
 (segment (start 115 86.24) (end 115 83.7) (width 0.25) (layer "F.Cu") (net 1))
 (segment (start 115.9175 117.7625) (end 115.9175 116.84) (width 0.25) (layer "F.Cu") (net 1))
 (segment (start 123.54 66.04) (end 121.92 67.66) (width 0.25) (layer "F.Cu") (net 1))
 (segment (start 129.145 70.725) (end 129.145 68.58) (width 0.25) (layer "F.Cu") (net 1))
 (segment (start 115 88.78) (end 115 86.24) (width 0.25) (layer "F.Cu") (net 1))
 (segment (start 115 81.16) (end 115 78.62) (width 0.25) (layer "F.Cu") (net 1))
 (segment (start 116.84 90.62) (end 115 88.78) (width 0.25) (layer "F.Cu") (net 1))
 (segment (start 113.3425 121.92) (end 113.3425 120.3375) (width 0.25) (layer "F.Cu") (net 1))
 (segment (start 134.62 71.2) (end 129.62 71.2) (width 0.25) (layer "F.Cu") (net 1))
 (segment (start 129.62 71.2) (end 129.145 70.725) (width 0.25) (layer "F.Cu") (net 1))
 (segment (start 112.621117 73.54) (end 115 73.54) (width 0.25) (layer "F.Cu") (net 1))
 (segment (start 126.605 66.04) (end 123.54 66.04) (width 0.25) (layer "F.Cu") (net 1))
 (segment (start 115.22 67.66) (end 112.26 70.62) (width 0.25) (layer "F.Cu") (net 1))
 (segment (start 113.3425 120.3375) (end 115.9175 117.7625) (width 0.25) (layer "F.Cu") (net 1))
 (segment (start 115 73.54) (end 115 76.08) (width 0.25) (layer "F.Cu") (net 1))
 (segment (start 121.92 67.66) (end 115.22 67.66) (width 0.25) (layer "F.Cu") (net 1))
 (segment (start 127 67.193409) (end 124.579533 64.772942) (width 0.25) (layer "B.Cu") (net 1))
 (segment (start 138.6325 87.63) (end 131.3275 80.325) (width 0.25) (layer "B.Cu") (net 1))
 (segment (start 131.3275 80.325) (end 129.657563 80.325) (width 0.25) (layer "B.Cu") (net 1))
 (segment (start 129.657563 80.325) (end 127 77.667437) (width 0.25) (layer "B.Cu") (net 1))
 (segment (start 139.24 87.63) (end 138.6325 87.63) (width 0.25) (layer "B.Cu") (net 1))
 (segment (start 127 77.667437) (end 127 67.193409) (width 0.25) (layer "B.Cu") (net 1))
 (segment (start 136.412894 70.442665) (end 136.412894 71.907106) (width 0.25) (layer "F.Cu") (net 7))
 (segment (start 111.76 91.44) (end 111.76 68.58) (width 0.25) (layer "F.Cu") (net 7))
 (segment (start 111.76 68.58) (end 114.3 66.04) (width 0.25) (layer "F.Cu") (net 7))
 (segment (start 136.412894 71.907106) (end 134.62 73.7) (width 0.25) (layer "F.Cu") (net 7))
 (segment (start 114.3 101.6) (end 114.3 93.98) (width 0.25) (layer "F.Cu") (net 7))
 (segment (start 134.62 68.649771) (end 136.412894 70.442665) (width 0.25) (layer "F.Cu") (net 7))
 (segment (start 114.3 66.04) (end 119.38 66.04) (width 0.25) (layer "F.Cu") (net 7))
 (segment (start 119.38 66.04) (end 122.978147 62.441853) (width 0.25) (layer "F.Cu") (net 7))
 (segment (start 114.3 93.98) (end 111.76 91.44) (width 0.25) (layer "F.Cu") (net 7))
 (segment (start 122.978147 62.441853) (end 128.481853 62.441853) (width 0.25) (layer "F.Cu") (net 7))
 (segment (start 134.62 68.58) (end 134.62 68.649771) (width 0.25) (layer "F.Cu") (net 7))
 (segment (start 128.481853 62.441853) (end 134.62 68.58) (width 0.25) (layer "F.Cu") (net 7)))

